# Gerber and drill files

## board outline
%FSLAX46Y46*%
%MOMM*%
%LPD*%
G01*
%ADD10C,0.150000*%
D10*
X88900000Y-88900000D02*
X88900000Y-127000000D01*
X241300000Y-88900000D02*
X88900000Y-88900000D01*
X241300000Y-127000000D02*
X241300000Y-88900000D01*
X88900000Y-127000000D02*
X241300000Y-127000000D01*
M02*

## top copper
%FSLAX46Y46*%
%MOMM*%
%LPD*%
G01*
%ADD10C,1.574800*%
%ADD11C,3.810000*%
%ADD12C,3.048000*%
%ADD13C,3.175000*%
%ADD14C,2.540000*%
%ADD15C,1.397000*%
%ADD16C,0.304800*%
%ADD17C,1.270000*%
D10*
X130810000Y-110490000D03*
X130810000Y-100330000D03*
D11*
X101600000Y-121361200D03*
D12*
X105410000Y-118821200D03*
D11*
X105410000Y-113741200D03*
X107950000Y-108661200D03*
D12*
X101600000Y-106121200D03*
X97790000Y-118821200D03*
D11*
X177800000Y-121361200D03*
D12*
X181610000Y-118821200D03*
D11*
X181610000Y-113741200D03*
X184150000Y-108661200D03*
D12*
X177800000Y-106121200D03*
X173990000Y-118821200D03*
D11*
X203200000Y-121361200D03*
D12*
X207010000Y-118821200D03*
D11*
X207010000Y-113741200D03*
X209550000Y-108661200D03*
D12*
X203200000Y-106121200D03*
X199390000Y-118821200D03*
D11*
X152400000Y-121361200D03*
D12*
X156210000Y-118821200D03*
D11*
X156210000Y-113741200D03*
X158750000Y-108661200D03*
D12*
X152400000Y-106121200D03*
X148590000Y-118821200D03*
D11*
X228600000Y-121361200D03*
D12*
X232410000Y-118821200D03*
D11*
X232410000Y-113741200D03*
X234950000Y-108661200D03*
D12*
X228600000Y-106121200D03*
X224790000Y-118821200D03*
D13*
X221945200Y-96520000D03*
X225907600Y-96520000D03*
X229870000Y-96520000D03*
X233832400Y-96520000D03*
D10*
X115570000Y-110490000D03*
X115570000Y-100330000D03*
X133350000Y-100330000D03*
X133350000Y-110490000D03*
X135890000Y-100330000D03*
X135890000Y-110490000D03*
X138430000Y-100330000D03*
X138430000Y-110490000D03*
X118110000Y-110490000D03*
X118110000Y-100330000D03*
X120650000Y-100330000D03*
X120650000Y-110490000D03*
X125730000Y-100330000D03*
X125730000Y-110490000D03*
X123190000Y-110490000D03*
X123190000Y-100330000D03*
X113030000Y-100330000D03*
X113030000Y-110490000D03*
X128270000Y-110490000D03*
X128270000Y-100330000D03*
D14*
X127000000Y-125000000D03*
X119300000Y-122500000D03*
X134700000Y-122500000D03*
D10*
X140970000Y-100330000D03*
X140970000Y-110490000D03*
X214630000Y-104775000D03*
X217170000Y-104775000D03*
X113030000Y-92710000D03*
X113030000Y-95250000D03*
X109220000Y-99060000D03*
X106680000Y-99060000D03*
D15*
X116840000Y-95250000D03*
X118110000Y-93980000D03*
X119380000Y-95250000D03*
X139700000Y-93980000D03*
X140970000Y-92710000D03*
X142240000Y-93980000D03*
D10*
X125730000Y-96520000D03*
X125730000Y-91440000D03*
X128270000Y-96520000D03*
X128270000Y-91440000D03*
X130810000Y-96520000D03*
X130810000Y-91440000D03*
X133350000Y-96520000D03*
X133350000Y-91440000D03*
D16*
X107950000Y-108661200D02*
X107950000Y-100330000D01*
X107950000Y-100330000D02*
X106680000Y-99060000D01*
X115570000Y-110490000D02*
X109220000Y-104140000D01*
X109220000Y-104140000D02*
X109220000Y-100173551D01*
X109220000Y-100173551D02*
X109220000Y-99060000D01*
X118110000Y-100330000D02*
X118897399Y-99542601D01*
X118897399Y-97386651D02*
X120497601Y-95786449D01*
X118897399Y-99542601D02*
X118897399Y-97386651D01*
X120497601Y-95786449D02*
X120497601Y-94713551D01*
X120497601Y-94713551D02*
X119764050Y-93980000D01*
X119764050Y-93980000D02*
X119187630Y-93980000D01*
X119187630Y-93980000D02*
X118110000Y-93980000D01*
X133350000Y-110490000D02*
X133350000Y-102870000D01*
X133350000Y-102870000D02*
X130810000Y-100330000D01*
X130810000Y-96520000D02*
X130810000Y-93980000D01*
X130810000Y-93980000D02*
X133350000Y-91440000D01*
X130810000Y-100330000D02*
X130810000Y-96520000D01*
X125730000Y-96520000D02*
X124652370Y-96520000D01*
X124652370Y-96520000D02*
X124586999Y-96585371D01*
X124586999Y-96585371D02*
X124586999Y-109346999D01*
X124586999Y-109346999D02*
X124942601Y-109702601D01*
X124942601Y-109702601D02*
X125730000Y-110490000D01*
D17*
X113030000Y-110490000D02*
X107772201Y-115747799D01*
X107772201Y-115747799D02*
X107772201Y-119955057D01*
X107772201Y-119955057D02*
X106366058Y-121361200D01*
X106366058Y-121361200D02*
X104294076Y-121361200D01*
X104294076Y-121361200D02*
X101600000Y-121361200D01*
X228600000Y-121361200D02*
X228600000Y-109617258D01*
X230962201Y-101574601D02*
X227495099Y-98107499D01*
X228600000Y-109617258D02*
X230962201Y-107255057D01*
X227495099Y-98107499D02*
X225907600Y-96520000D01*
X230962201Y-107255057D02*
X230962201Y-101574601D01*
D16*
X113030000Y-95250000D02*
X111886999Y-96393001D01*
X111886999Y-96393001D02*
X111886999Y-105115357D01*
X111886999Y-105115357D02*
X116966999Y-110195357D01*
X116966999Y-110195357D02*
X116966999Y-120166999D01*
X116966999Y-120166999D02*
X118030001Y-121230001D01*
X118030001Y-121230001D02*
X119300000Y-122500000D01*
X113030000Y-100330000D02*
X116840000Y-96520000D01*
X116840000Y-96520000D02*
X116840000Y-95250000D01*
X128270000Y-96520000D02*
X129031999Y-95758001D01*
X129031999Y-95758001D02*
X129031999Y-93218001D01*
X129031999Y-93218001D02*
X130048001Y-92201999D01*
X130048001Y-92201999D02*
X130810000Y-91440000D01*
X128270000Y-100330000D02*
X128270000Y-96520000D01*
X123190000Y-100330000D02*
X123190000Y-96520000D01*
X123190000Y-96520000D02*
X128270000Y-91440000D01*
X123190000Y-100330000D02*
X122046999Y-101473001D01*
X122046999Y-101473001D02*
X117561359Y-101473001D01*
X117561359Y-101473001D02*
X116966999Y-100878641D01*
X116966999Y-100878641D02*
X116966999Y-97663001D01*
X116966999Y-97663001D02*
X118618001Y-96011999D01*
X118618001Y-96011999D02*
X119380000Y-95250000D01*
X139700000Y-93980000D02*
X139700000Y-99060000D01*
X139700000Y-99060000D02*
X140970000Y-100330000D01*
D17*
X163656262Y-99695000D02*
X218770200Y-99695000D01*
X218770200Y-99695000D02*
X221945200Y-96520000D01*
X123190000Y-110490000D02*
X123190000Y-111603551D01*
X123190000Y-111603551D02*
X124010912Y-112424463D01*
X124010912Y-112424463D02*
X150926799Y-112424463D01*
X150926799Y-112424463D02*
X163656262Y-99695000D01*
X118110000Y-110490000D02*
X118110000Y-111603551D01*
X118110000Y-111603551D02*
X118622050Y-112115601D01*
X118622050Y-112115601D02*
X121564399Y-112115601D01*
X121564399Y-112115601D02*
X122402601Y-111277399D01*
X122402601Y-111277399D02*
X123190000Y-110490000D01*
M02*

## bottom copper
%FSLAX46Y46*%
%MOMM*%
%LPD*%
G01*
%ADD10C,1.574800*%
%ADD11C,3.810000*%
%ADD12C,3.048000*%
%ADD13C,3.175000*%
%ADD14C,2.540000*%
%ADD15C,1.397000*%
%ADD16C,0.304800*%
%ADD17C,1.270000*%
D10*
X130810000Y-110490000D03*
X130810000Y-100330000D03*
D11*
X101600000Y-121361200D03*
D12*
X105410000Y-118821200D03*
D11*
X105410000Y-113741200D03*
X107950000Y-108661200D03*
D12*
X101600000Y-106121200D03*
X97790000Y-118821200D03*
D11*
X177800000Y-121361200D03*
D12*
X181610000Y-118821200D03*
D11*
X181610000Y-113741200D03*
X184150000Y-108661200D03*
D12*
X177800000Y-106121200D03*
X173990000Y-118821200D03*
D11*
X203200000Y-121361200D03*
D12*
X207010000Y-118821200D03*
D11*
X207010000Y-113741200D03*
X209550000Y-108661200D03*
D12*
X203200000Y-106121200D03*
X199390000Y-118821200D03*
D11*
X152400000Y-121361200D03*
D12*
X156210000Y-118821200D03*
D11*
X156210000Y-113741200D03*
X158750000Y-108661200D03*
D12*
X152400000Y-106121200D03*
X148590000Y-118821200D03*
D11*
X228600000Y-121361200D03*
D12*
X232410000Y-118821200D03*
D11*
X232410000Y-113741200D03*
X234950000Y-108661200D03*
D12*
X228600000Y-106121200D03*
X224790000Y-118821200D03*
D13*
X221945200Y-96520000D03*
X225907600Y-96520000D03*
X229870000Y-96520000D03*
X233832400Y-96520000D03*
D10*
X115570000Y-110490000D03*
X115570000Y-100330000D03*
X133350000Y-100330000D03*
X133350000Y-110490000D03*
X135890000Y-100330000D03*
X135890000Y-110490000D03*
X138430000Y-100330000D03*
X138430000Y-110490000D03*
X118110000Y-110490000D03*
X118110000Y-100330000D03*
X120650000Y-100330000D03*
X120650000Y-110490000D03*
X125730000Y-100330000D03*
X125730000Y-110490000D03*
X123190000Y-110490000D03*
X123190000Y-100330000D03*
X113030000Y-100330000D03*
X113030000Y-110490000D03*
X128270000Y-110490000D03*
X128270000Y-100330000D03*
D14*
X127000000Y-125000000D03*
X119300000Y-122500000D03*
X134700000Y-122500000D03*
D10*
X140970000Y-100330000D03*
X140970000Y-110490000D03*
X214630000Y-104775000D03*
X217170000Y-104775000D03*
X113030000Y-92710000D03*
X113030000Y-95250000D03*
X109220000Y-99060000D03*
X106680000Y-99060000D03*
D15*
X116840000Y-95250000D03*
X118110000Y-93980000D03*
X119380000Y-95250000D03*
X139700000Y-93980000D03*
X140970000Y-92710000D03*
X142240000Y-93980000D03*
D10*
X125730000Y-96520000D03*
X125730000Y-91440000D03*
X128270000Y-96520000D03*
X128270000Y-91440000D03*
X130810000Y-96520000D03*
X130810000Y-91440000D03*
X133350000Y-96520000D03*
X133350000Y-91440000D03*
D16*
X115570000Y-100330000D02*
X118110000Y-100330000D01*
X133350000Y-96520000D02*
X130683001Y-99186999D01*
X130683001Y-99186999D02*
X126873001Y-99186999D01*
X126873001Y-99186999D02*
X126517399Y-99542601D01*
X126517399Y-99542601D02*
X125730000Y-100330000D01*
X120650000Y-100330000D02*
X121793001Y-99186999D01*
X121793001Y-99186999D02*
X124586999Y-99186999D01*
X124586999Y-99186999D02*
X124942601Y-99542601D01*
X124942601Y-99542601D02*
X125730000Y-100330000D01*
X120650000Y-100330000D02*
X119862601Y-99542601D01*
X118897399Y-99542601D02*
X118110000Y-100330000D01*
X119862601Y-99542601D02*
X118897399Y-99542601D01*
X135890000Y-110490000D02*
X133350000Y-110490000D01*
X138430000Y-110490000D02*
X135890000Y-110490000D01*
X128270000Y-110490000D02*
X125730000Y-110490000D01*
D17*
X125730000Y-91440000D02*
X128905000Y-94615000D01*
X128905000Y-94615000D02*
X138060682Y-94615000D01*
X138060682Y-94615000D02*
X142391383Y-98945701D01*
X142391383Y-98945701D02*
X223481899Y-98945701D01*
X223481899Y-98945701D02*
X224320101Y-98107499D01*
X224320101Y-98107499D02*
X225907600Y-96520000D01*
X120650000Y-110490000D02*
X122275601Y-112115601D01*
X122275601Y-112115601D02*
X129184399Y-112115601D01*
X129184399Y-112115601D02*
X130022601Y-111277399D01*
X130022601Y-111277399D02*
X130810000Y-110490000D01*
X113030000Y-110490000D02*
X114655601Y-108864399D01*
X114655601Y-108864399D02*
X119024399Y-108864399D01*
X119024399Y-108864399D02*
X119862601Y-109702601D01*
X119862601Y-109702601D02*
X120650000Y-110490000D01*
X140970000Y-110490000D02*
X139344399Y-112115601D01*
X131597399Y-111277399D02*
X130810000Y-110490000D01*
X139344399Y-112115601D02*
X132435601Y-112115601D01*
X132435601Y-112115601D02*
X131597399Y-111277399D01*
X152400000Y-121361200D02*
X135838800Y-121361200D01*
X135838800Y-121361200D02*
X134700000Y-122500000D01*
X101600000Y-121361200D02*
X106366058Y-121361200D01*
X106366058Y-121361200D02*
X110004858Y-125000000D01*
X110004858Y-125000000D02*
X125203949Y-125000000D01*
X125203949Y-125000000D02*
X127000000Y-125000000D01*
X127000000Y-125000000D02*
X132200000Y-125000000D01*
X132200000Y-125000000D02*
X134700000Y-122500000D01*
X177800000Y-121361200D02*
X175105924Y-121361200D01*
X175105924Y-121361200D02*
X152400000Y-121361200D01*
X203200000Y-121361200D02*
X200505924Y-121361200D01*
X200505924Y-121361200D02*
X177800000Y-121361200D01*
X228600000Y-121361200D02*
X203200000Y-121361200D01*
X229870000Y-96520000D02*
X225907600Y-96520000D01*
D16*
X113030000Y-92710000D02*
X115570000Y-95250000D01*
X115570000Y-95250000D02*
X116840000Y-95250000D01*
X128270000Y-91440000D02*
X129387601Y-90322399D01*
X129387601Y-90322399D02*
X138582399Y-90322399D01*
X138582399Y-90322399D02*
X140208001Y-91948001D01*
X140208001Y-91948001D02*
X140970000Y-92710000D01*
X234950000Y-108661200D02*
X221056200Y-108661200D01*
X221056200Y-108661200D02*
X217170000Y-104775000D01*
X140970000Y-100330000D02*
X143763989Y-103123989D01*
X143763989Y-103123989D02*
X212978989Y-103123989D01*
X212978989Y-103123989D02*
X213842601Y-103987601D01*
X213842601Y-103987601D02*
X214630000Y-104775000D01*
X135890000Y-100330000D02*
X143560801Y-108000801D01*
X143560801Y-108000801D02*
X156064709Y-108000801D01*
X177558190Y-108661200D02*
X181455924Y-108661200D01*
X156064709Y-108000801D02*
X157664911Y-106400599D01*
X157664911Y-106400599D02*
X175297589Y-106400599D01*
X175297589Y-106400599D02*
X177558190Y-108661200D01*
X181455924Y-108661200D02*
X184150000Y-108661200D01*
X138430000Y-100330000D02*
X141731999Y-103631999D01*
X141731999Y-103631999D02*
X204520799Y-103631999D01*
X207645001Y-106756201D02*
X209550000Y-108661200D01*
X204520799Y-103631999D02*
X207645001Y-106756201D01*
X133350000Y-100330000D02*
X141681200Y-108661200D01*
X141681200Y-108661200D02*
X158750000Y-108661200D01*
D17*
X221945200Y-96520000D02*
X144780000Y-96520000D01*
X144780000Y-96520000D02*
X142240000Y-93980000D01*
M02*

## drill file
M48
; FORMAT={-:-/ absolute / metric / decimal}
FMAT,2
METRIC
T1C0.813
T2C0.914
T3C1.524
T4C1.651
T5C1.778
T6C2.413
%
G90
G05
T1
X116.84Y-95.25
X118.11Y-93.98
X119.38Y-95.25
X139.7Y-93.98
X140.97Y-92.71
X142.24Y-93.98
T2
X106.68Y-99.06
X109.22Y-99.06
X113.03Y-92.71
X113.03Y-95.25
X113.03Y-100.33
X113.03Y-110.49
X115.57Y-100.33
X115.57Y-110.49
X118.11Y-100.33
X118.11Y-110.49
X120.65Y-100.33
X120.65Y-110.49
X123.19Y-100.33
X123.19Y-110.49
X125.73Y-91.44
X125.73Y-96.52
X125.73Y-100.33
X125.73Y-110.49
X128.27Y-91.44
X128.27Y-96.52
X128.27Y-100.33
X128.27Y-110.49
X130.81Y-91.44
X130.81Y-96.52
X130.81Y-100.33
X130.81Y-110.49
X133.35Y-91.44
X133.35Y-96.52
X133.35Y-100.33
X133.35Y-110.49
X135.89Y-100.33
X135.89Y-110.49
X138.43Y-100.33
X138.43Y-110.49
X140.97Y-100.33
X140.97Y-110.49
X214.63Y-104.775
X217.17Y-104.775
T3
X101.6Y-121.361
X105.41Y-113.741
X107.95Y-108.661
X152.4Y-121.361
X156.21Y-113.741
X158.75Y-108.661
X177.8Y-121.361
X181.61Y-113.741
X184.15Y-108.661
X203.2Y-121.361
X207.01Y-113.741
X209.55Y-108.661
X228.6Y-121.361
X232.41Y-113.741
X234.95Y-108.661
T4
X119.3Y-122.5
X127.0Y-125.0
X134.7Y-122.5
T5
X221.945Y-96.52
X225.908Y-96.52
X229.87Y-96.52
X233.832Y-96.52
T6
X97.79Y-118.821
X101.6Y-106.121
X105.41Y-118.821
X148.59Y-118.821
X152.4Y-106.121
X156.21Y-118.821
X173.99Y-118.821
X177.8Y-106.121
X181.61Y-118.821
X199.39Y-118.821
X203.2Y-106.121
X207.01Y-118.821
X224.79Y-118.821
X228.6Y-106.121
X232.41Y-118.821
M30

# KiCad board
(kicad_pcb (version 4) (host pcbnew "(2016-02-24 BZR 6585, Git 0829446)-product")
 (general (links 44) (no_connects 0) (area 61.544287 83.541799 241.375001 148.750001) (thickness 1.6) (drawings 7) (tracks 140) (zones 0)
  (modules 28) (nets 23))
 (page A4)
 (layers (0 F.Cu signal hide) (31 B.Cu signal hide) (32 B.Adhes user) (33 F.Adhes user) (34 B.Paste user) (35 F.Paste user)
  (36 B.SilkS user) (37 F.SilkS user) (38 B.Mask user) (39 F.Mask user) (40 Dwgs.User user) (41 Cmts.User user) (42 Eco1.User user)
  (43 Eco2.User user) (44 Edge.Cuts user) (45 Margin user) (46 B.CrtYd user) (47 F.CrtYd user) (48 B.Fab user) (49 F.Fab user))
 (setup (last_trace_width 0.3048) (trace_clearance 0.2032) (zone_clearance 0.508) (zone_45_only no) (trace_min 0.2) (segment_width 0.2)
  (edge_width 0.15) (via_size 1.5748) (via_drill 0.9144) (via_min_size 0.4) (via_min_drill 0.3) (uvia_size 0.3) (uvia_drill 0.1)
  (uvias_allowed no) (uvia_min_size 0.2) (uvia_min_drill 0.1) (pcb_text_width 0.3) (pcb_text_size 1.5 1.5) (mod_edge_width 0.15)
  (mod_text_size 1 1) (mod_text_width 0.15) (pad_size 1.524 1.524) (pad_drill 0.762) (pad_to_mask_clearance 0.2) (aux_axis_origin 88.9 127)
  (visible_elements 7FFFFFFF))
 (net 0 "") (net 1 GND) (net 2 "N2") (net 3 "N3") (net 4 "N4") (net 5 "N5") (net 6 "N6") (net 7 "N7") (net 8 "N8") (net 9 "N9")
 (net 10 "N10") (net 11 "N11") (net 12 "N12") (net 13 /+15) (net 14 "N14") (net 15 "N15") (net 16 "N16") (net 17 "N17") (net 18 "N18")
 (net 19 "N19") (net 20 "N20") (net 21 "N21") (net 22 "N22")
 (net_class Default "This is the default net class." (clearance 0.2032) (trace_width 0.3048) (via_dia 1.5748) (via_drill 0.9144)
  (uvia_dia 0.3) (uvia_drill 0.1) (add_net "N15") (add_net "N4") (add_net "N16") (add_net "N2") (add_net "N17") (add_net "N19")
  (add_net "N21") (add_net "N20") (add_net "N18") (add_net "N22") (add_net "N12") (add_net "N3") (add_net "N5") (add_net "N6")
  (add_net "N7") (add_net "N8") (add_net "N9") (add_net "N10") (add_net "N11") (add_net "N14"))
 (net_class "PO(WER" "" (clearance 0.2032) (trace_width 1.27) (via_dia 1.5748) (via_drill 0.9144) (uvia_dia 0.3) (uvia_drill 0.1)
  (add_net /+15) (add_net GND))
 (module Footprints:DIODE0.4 (layer F.Cu) (at 130.81 105.41 90)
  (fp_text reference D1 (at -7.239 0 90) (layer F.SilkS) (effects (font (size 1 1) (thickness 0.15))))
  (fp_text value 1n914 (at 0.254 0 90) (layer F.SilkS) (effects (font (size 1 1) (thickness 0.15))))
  (pad 1 thru_hole circle (at -5.08 0 90) (size 1.5748 1.5748) (drill 0.9144) (layers *.Cu *.Mask F.SilkS) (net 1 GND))
  (pad 2 thru_hole circle (at 5.08 0 90) (size 1.5748 1.5748) (drill 0.9144) (layers *.Cu *.Mask F.SilkS) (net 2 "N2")))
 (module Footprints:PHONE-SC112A (layer F.Cu) (at 101.6 127 270)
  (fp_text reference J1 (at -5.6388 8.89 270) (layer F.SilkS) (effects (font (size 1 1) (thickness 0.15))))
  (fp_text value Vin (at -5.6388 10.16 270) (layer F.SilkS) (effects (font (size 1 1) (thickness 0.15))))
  (pad 1 thru_hole circle (at -5.6388 0 270) (size 3.81 3.81) (drill 1.524) (layers *.Cu *.Mask F.SilkS) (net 1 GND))
  (pad "" thru_hole circle (at -8.1788 -3.81 270) (size 3.048 3.048) (drill 2.413) (layers *.Cu *.Mask F.SilkS))
  (pad 2 thru_hole circle (at -13.2588 -3.81 270) (size 3.81 3.81) (drill 1.524) (layers *.Cu *.Mask F.SilkS) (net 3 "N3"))
  (pad 3 thru_hole circle (at -18.3388 -6.35 270) (size 3.81 3.81) (drill 1.524) (layers *.Cu *.Mask F.SilkS) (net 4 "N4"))
  (pad "" thru_hole circle (at -20.8788 0 270) (size 3.048 3.048) (drill 2.413) (layers *.Cu *.Mask F.SilkS))
  (pad "" thru_hole circle (at -8.1788 3.81 270) (size 3.048 3.048) (drill 2.413) (layers *.Cu *.Mask F.SilkS)))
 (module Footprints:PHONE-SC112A (layer F.Cu) (at 177.8 127 270)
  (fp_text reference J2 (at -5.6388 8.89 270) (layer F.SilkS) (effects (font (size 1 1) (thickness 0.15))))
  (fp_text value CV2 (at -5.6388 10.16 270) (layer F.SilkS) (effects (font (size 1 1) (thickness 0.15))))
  (pad 1 thru_hole circle (at -5.6388 0 270) (size 3.81 3.81) (drill 1.524) (layers *.Cu *.Mask F.SilkS) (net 1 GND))
  (pad "" thru_hole circle (at -8.1788 -3.81 270) (size 3.048 3.048) (drill 2.413) (layers *.Cu *.Mask F.SilkS))
  (pad 2 thru_hole circle (at -13.2588 -3.81 270) (size 3.81 3.81) (drill 1.524) (layers *.Cu *.Mask F.SilkS) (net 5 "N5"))
  (pad 3 thru_hole circle (at -18.3388 -6.35 270) (size 3.81 3.81) (drill 1.524) (layers *.Cu *.Mask F.SilkS) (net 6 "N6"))
  (pad "" thru_hole circle (at -20.8788 0 270) (size 3.048 3.048) (drill 2.413) (layers *.Cu *.Mask F.SilkS))
  (pad "" thru_hole circle (at -8.1788 3.81 270) (size 3.048 3.048) (drill 2.413) (layers *.Cu *.Mask F.SilkS)))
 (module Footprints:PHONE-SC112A (layer F.Cu) (at 203.2 127 270)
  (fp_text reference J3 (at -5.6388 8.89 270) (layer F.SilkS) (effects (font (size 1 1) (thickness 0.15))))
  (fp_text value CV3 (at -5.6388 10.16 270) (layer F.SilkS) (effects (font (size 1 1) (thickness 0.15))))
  (pad 1 thru_hole circle (at -5.6388 0 270) (size 3.81 3.81) (drill 1.524) (layers *.Cu *.Mask F.SilkS) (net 1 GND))
  (pad "" thru_hole circle (at -8.1788 -3.81 270) (size 3.048 3.048) (drill 2.413) (layers *.Cu *.Mask F.SilkS))
  (pad 2 thru_hole circle (at -13.2588 -3.81 270) (size 3.81 3.81) (drill 1.524) (layers *.Cu *.Mask F.SilkS) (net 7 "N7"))
  (pad 3 thru_hole circle (at -18.3388 -6.35 270) (size 3.81 3.81) (drill 1.524) (layers *.Cu *.Mask F.SilkS) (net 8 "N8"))
  (pad "" thru_hole circle (at -20.8788 0 270) (size 3.048 3.048) (drill 2.413) (layers *.Cu *.Mask F.SilkS))
  (pad "" thru_hole circle (at -8.1788 3.81 270) (size 3.048 3.048) (drill 2.413) (layers *.Cu *.Mask F.SilkS)))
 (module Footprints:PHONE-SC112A (layer F.Cu) (at 152.4 127 270)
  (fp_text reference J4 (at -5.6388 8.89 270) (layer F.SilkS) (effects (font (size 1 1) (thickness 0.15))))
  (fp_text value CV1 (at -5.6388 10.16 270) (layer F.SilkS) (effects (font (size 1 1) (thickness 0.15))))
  (pad 1 thru_hole circle (at -5.6388 0 270) (size 3.81 3.81) (drill 1.524) (layers *.Cu *.Mask F.SilkS) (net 1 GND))
  (pad "" thru_hole circle (at -8.1788 -3.81 270) (size 3.048 3.048) (drill 2.413) (layers *.Cu *.Mask F.SilkS))
  (pad 2 thru_hole circle (at -13.2588 -3.81 270) (size 3.81 3.81) (drill 1.524) (layers *.Cu *.Mask F.SilkS) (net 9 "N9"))
  (pad 3 thru_hole circle (at -18.3388 -6.35 270) (size 3.81 3.81) (drill 1.524) (layers *.Cu *.Mask F.SilkS) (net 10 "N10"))
  (pad "" thru_hole circle (at -20.8788 0 270) (size 3.048 3.048) (drill 2.413) (layers *.Cu *.Mask F.SilkS))
  (pad "" thru_hole circle (at -8.1788 3.81 270) (size 3.048 3.048) (drill 2.413) (layers *.Cu *.Mask F.SilkS)))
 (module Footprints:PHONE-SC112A (layer F.Cu) (at 228.6 127 270)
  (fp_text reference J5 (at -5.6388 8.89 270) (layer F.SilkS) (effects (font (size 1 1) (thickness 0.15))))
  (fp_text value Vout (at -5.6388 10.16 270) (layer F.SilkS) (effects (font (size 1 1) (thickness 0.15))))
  (pad 1 thru_hole circle (at -5.6388 0 270) (size 3.81 3.81) (drill 1.524) (layers *.Cu *.Mask F.SilkS) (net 1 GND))
  (pad "" thru_hole circle (at -8.1788 -3.81 270) (size 3.048 3.048) (drill 2.413) (layers *.Cu *.Mask F.SilkS))
  (pad 2 thru_hole circle (at -13.2588 -3.81 270) (size 3.81 3.81) (drill 1.524) (layers *.Cu *.Mask F.SilkS) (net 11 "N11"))
  (pad 3 thru_hole circle (at -18.3388 -6.35 270) (size 3.81 3.81) (drill 1.524) (layers *.Cu *.Mask F.SilkS) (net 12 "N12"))
  (pad "" thru_hole circle (at -20.8788 0 270) (size 3.048 3.048) (drill 2.413) (layers *.Cu *.Mask F.SilkS))
  (pad "" thru_hole circle (at -8.1788 3.81 270) (size 3.048 3.048) (drill 2.413) (layers *.Cu *.Mask F.SilkS)))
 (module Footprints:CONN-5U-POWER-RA (layer F.Cu) (at 227.8888 96.52)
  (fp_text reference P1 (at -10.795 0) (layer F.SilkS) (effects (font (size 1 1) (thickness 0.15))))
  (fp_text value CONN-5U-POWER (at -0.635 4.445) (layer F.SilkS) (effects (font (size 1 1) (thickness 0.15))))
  (pad 1 thru_hole circle (at -5.9436 0) (size 3.175 3.175) (drill 1.778) (layers *.Cu *.Mask F.SilkS) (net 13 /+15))
  (pad 2 thru_hole circle (at -1.9812 0) (size 3.175 3.175) (drill 1.778) (layers *.Cu *.Mask F.SilkS) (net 1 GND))
  (pad 3 thru_hole circle (at 1.9812 0) (size 3.175 3.175) (drill 1.778) (layers *.Cu *.Mask F.SilkS) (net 1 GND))
  (pad 4 thru_hole circle (at 5.9436 0) (size 3.175 3.175) (drill 1.778) (layers *.Cu *.Mask F.SilkS) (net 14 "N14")))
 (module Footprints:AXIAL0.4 (layer F.Cu) (at 115.57 105.41 90)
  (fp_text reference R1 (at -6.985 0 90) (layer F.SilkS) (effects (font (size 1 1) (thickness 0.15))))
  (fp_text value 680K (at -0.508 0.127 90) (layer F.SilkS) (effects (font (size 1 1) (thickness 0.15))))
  (pad 1 thru_hole circle (at -5.08 0 90) (size 1.5748 1.5748) (drill 0.9144) (layers *.Cu *.Mask F.SilkS) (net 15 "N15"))
  (pad 2 thru_hole circle (at 5.08 0 90) (size 1.5748 1.5748) (drill 0.9144) (layers *.Cu *.Mask F.SilkS) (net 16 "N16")))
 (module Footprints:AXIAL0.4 (layer F.Cu) (at 133.35 105.41 270)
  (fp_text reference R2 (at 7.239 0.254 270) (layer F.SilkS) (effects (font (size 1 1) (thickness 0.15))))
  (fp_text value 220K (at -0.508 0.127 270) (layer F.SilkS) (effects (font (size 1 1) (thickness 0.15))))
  (pad 1 thru_hole circle (at -5.08 0 270) (size 1.5748 1.5748) (drill 0.9144) (layers *.Cu *.Mask F.SilkS) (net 10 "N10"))
  (pad 2 thru_hole circle (at 5.08 0 270) (size 1.5748 1.5748) (drill 0.9144) (layers *.Cu *.Mask F.SilkS) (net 2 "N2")))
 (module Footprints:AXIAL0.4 (layer F.Cu) (at 135.89 105.41 270)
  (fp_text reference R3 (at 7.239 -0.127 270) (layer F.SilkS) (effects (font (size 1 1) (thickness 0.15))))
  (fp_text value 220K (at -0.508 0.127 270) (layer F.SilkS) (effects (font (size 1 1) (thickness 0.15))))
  (pad 1 thru_hole circle (at -5.08 0 270) (size 1.5748 1.5748) (drill 0.9144) (layers *.Cu *.Mask F.SilkS) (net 6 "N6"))
  (pad 2 thru_hole circle (at 5.08 0 270) (size 1.5748 1.5748) (drill 0.9144) (layers *.Cu *.Mask F.SilkS) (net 2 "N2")))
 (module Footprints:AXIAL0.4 (layer F.Cu) (at 138.43 105.41 270)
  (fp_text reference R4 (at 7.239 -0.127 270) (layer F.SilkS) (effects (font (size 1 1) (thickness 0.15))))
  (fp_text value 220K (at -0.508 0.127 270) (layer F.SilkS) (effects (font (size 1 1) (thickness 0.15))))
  (pad 1 thru_hole circle (at -5.08 0 270) (size 1.5748 1.5748) (drill 0.9144) (layers *.Cu *.Mask F.SilkS) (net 8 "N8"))
  (pad 2 thru_hole circle (at 5.08 0 270) (size 1.5748 1.5748) (drill 0.9144) (layers *.Cu *.Mask F.SilkS) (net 2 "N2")))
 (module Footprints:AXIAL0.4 (layer F.Cu) (at 118.11 105.41 90)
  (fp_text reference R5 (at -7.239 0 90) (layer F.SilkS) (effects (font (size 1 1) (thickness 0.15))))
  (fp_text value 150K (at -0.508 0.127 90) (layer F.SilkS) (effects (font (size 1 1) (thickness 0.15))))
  (pad 1 thru_hole circle (at -5.08 0 90) (size 1.5748 1.5748) (drill 0.9144) (layers *.Cu *.Mask F.SilkS) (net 13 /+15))
  (pad 2 thru_hole circle (at 5.08 0 90) (size 1.5748 1.5748) (drill 0.9144) (layers *.Cu *.Mask F.SilkS) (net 16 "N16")))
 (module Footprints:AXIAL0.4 (layer F.Cu) (at 120.65 105.41 270)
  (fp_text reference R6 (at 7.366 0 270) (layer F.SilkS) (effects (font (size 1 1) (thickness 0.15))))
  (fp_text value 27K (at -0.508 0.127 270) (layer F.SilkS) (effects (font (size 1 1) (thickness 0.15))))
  (pad 1 thru_hole circle (at -5.08 0 270) (size 1.5748 1.5748) (drill 0.9144) (layers *.Cu *.Mask F.SilkS) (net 16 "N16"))
  (pad 2 thru_hole circle (at 5.08 0 270) (size 1.5748 1.5748) (drill 0.9144) (layers *.Cu *.Mask F.SilkS) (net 1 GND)))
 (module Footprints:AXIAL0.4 (layer F.Cu) (at 125.73 105.41 270)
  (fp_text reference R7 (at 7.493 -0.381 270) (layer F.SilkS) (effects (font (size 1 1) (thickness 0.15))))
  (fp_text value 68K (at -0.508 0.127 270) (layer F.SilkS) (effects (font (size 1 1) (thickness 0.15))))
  (pad 1 thru_hole circle (at -5.08 0 270) (size 1.5748 1.5748) (drill 0.9144) (layers *.Cu *.Mask F.SilkS) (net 16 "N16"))
  (pad 2 thru_hole circle (at 5.08 0 270) (size 1.5748 1.5748) (drill 0.9144) (layers *.Cu *.Mask F.SilkS) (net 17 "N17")))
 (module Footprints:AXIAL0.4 (layer F.Cu) (at 123.19 105.41 90)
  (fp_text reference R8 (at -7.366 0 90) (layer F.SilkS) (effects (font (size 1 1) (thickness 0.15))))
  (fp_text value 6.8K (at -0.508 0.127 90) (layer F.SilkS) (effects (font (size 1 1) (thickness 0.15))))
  (pad 1 thru_hole circle (at -5.08 0 90) (size 1.5748 1.5748) (drill 0.9144) (layers *.Cu *.Mask F.SilkS) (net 13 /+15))
  (pad 2 thru_hole circle (at 5.08 0 90) (size 1.5748 1.5748) (drill 0.9144) (layers *.Cu *.Mask F.SilkS) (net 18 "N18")))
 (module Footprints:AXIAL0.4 (layer F.Cu) (at 113.03 105.41 270)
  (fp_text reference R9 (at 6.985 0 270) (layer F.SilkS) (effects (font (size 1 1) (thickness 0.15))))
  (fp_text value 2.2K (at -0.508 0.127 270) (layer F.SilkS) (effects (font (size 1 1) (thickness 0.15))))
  (pad 1 thru_hole circle (at -5.08 0 270) (size 1.5748 1.5748) (drill 0.9144) (layers *.Cu *.Mask F.SilkS) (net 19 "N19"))
  (pad 2 thru_hole circle (at 5.08 0 270) (size 1.5748 1.5748) (drill 0.9144) (layers *.Cu *.Mask F.SilkS) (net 1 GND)))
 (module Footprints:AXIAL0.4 (layer F.Cu) (at 128.27 105.41 90)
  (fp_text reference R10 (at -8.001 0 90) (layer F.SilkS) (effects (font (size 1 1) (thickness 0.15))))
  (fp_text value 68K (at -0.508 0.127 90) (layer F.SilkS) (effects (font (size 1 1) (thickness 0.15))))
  (pad 1 thru_hole circle (at -5.08 0 90) (size 1.5748 1.5748) (drill 0.9144) (layers *.Cu *.Mask F.SilkS) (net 17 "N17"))
  (pad 2 thru_hole circle (at 5.08 0 90) (size 1.5748 1.5748) (drill 0.9144) (layers *.Cu *.Mask F.SilkS) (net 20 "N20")))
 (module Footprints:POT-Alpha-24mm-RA (layer F.Cu) (at 127 127)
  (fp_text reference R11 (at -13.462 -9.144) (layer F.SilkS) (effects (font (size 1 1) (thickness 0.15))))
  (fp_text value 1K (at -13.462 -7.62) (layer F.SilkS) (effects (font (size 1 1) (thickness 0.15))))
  (pad 2 thru_hole circle (at 0 -2) (size 2.54 2.54) (drill 1.651) (layers *.Cu *.Mask F.SilkS) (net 1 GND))
  (pad 1 thru_hole circle (at -7.7 -4.5) (size 2.54 2.54) (drill 1.651) (layers *.Cu *.Mask F.SilkS) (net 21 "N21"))
  (pad 3 thru_hole circle (at 7.7 -4.5) (size 2.54 2.54) (drill 1.651) (layers *.Cu *.Mask F.SilkS) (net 1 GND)))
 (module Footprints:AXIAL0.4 (layer F.Cu) (at 140.97 105.41 270)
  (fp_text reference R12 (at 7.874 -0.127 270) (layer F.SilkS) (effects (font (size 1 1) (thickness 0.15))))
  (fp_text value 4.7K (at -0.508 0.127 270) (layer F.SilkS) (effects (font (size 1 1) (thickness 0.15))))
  (pad 1 thru_hole circle (at -5.08 0 270) (size 1.5748 1.5748) (drill 0.9144) (layers *.Cu *.Mask F.SilkS) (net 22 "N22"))
  (pad 2 thru_hole circle (at 5.08 0 270) (size 1.5748 1.5748) (drill 0.9144) (layers *.Cu *.Mask F.SilkS) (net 1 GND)))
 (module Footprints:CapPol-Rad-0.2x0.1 (layer F.Cu) (at 217.17 107.315)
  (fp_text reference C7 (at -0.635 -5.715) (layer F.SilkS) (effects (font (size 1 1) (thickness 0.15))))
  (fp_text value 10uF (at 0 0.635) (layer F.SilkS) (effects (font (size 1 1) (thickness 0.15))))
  (pad 1 thru_hole circle (at -2.54 -2.54) (size 1.5748 1.5748) (drill 0.9144) (layers *.Cu *.Mask F.SilkS) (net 22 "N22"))
  (pad 2 thru_hole circle (at 0 -2.54) (size 1.5748 1.5748) (drill 0.9144) (layers *.Cu *.Mask F.SilkS) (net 12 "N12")))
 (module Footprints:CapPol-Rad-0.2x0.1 (layer F.Cu) (at 110.49 95.25 270)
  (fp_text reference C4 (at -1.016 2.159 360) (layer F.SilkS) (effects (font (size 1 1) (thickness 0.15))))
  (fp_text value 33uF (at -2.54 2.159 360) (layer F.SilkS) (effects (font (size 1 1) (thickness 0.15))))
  (pad 1 thru_hole circle (at -2.54 -2.54 270) (size 1.5748 1.5748) (drill 0.9144) (layers *.Cu *.Mask F.SilkS) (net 19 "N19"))
  (pad 2 thru_hole circle (at 0 -2.54 270) (size 1.5748 1.5748) (drill 0.9144) (layers *.Cu *.Mask F.SilkS) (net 21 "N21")))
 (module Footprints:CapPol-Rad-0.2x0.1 (layer F.Cu) (at 106.68 96.52 180)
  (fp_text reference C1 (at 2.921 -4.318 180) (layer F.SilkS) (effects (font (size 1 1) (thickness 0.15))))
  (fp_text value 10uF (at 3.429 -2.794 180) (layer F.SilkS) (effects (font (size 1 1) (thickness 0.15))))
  (pad 1 thru_hole circle (at -2.54 -2.54 180) (size 1.5748 1.5748) (drill 0.9144) (layers *.Cu *.Mask F.SilkS) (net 15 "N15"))
  (pad 2 thru_hole circle (at 0 -2.54 180) (size 1.5748 1.5748) (drill 0.9144) (layers *.Cu *.Mask F.SilkS) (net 4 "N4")))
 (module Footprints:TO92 (layer F.Cu) (at 118.11 97.79)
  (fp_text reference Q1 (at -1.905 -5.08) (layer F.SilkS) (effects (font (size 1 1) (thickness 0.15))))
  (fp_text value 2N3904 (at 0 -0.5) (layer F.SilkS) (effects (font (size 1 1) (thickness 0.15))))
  (pad 1 thru_hole circle (at -1.27 -2.54) (size 1.397 1.397) (drill 0.8128) (layers *.Cu *.Mask F.SilkS) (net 19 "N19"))
  (pad 2 thru_hole circle (at 0 -3.81) (size 1.397 1.397) (drill 0.8128) (layers *.Cu *.Mask F.SilkS) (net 16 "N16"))
  (pad 3 thru_hole circle (at 1.27 -2.54) (size 1.397 1.397) (drill 0.8128) (layers *.Cu *.Mask F.SilkS) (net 18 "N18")))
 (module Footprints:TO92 (layer F.Cu) (at 140.97 96.52)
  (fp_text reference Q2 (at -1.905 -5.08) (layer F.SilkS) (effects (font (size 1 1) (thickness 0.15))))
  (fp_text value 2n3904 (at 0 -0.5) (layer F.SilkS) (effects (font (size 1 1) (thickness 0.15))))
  (pad 1 thru_hole circle (at -1.27 -2.54) (size 1.397 1.397) (drill 0.8128) (layers *.Cu *.Mask F.SilkS) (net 22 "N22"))
  (pad 2 thru_hole circle (at 0 -3.81) (size 1.397 1.397) (drill 0.8128) (layers *.Cu *.Mask F.SilkS) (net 18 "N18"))
  (pad 3 thru_hole circle (at 1.27 -2.54) (size 1.397 1.397) (drill 0.8128) (layers *.Cu *.Mask F.SilkS) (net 13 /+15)))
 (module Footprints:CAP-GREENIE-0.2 (layer F.Cu) (at 125.73 93.98 90)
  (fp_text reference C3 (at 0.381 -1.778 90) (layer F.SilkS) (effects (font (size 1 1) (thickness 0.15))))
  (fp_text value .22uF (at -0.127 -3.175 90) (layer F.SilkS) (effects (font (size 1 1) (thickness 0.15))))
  (pad 1 thru_hole circle (at -2.54 0 90) (size 1.5748 1.5748) (drill 0.9144) (layers *.Cu *.Mask F.SilkS) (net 17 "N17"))
  (pad 2 thru_hole circle (at 2.54 0 90) (size 1.5748 1.5748) (drill 0.9144) (layers *.Cu *.Mask F.SilkS) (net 1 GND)))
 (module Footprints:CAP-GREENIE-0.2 (layer F.Cu) (at 128.27 93.98 90)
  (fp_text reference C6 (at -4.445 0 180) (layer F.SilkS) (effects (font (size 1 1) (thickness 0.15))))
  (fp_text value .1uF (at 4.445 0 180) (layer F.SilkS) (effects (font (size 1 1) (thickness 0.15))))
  (pad 1 thru_hole circle (at -2.54 0 90) (size 1.5748 1.5748) (drill 0.9144) (layers *.Cu *.Mask F.SilkS) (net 20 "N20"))
  (pad 2 thru_hole circle (at 2.54 0 90) (size 1.5748 1.5748) (drill 0.9144) (layers *.Cu *.Mask F.SilkS) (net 18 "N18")))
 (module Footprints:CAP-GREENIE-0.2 (layer F.Cu) (at 130.81 93.98 90)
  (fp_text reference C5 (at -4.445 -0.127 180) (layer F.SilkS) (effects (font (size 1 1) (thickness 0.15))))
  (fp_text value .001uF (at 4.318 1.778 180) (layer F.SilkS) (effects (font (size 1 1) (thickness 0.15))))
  (pad 1 thru_hole circle (at -2.54 0 90) (size 1.5748 1.5748) (drill 0.9144) (layers *.Cu *.Mask F.SilkS) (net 2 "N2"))
  (pad 2 thru_hole circle (at 2.54 0 90) (size 1.5748 1.5748) (drill 0.9144) (layers *.Cu *.Mask F.SilkS) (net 20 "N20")))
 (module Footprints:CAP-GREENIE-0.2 (layer F.Cu) (at 133.35 93.98 90)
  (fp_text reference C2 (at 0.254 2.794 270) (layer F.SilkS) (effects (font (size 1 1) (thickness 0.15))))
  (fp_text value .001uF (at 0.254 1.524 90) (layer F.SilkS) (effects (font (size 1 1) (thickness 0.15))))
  (pad 1 thru_hole circle (at -2.54 0 90) (size 1.5748 1.5748) (drill 0.9144) (layers *.Cu *.Mask F.SilkS) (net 16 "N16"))
  (pad 2 thru_hole circle (at 2.54 0 90) (size 1.5748 1.5748) (drill 0.9144) (layers *.Cu *.Mask F.SilkS) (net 2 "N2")))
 (gr_line (start 88.9 88.9) (end 88.9 127) (layer Edge.Cuts) (width 0.15))
 (gr_line (start 241.3 88.9) (end 88.9 88.9) (layer Edge.Cuts) (width 0.15))
 (gr_line (start 241.3 127) (end 241.3 88.9) (layer Edge.Cuts) (width 0.15))
 (gr_line (start 88.9 127) (end 241.3 127) (layer Edge.Cuts) (width 0.15))
 (segment (start 107.95 108.6612) (end 107.95 100.33) (width 0.3048) (layer F.Cu) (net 4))
 (segment (start 107.95 100.33) (end 106.68 99.06) (width 0.3048) (layer F.Cu) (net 4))
 (segment (start 115.57 110.49) (end 109.22 104.14) (width 0.3048) (layer F.Cu) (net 15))
 (segment (start 109.22 104.14) (end 109.22 100.173551) (width 0.3048) (layer F.Cu) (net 15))
 (segment (start 109.22 100.173551) (end 109.22 99.06) (width 0.3048) (layer F.Cu) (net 15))
 (segment (start 115.57 100.33) (end 118.11 100.33) (width 0.3048) (layer B.Cu) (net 16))
 (segment (start 133.35 96.52) (end 130.683001 99.186999) (width 0.3048) (layer B.Cu) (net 16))
 (segment (start 130.683001 99.186999) (end 126.873001 99.186999) (width 0.3048) (layer B.Cu) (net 16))
 (segment (start 126.873001 99.186999) (end 126.517399 99.542601) (width 0.3048) (layer B.Cu) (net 16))
 (segment (start 126.517399 99.542601) (end 125.73 100.33) (width 0.3048) (layer B.Cu) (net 16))
 (segment (start 120.65 100.33) (end 121.793001 99.186999) (width 0.3048) (layer B.Cu) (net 16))
 (segment (start 121.793001 99.186999) (end 124.586999 99.186999) (width 0.3048) (layer B.Cu) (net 16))
 (segment (start 124.586999 99.186999) (end 124.942601 99.542601) (width 0.3048) (layer B.Cu) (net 16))
 (segment (start 124.942601 99.542601) (end 125.73 100.33) (width 0.3048) (layer B.Cu) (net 16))
 (segment (start 120.65 100.33) (end 119.862601 99.542601) (width 0.3048) (layer B.Cu) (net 16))
 (segment (start 118.897399 99.542601) (end 118.11 100.33) (width 0.3048) (layer B.Cu) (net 16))
 (segment (start 119.862601 99.542601) (end 118.897399 99.542601) (width 0.3048) (layer B.Cu) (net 16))
 (segment (start 118.11 100.33) (end 118.897399 99.542601) (width 0.3048) (layer F.Cu) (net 16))
 (segment (start 118.897399 97.386651) (end 120.497601 95.786449) (width 0.3048) (layer F.Cu) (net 16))
 (segment (start 118.897399 99.542601) (end 118.897399 97.386651) (width 0.3048) (layer F.Cu) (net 16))
 (segment (start 120.497601 95.786449) (end 120.497601 94.713551) (width 0.3048) (layer F.Cu) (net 16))
 (segment (start 120.497601 94.713551) (end 119.76405 93.98) (width 0.3048) (layer F.Cu) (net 16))
 (segment (start 119.76405 93.98) (end 119.18763 93.98) (width 0.3048) (layer F.Cu) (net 16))
 (segment (start 119.18763 93.98) (end 118.11 93.98) (width 0.3048) (layer F.Cu) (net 16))
 (segment (start 133.35 110.49) (end 133.35 102.87) (width 0.3048) (layer F.Cu) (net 2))
 (segment (start 133.35 102.87) (end 130.81 100.33) (width 0.3048) (layer F.Cu) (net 2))
 (segment (start 135.89 110.49) (end 133.35 110.49) (width 0.3048) (layer B.Cu) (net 2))
 (segment (start 138.43 110.49) (end 135.89 110.49) (width 0.3048) (layer B.Cu) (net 2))
 (segment (start 130.81 96.52) (end 130.81 93.98) (width 0.3048) (layer F.Cu) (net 2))
 (segment (start 130.81 93.98) (end 133.35 91.44) (width 0.3048) (layer F.Cu) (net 2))
 (segment (start 130.81 100.33) (end 130.81 96.52) (width 0.3048) (layer F.Cu) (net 2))
 (segment (start 128.27 110.49) (end 125.73 110.49) (width 0.3048) (layer B.Cu) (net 17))
 (segment (start 125.73 96.52) (end 124.65237 96.52) (width 0.3048) (layer F.Cu) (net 17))
 (segment (start 124.65237 96.52) (end 124.586999 96.585371) (width 0.3048) (layer F.Cu) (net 17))
 (segment (start 124.586999 96.585371) (end 124.586999 109.346999) (width 0.3048) (layer F.Cu) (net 17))
 (segment (start 124.586999 109.346999) (end 124.942601 109.702601) (width 0.3048) (layer F.Cu) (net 17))
 (segment (start 124.942601 109.702601) (end 125.73 110.49) (width 0.3048) (layer F.Cu) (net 17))
 (segment (start 125.73 91.44) (end 128.905 94.615) (width 1.27) (layer B.Cu) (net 1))
 (segment (start 128.905 94.615) (end 138.060682 94.615) (width 1.27) (layer B.Cu) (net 1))
 (segment (start 138.060682 94.615) (end 142.391383 98.945701) (width 1.27) (layer B.Cu) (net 1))
 (segment (start 142.391383 98.945701) (end 223.481899 98.945701) (width 1.27) (layer B.Cu) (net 1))
 (segment (start 223.481899 98.945701) (end 224.320101 98.107499) (width 1.27) (layer B.Cu) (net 1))
 (segment (start 224.320101 98.107499) (end 225.9076 96.52) (width 1.27) (layer B.Cu) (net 1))
 (segment (start 113.03 110.49) (end 107.772201 115.747799) (width 1.27) (layer F.Cu) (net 1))
 (segment (start 107.772201 115.747799) (end 107.772201 119.955057) (width 1.27) (layer F.Cu) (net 1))
 (segment (start 107.772201 119.955057) (end 106.366058 121.3612) (width 1.27) (layer F.Cu) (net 1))
 (segment (start 106.366058 121.3612) (end 104.294076 121.3612) (width 1.27) (layer F.Cu) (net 1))
 (segment (start 104.294076 121.3612) (end 101.6 121.3612) (width 1.27) (layer F.Cu) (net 1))
 (segment (start 120.65 110.49) (end 122.275601 112.115601) (width 1.27) (layer B.Cu) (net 1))
 (segment (start 122.275601 112.115601) (end 129.184399 112.115601) (width 1.27) (layer B.Cu) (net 1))
 (segment (start 129.184399 112.115601) (end 130.022601 111.277399) (width 1.27) (layer B.Cu) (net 1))
 (segment (start 130.022601 111.277399) (end 130.81 110.49) (width 1.27) (layer B.Cu) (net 1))
 (segment (start 113.03 110.49) (end 114.655601 108.864399) (width 1.27) (layer B.Cu) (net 1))
 (segment (start 114.655601 108.864399) (end 119.024399 108.864399) (width 1.27) (layer B.Cu) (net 1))
 (segment (start 119.024399 108.864399) (end 119.862601 109.702601) (width 1.27) (layer B.Cu) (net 1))
 (segment (start 119.862601 109.702601) (end 120.65 110.49) (width 1.27) (layer B.Cu) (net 1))
 (segment (start 140.97 110.49) (end 139.344399 112.115601) (width 1.27) (layer B.Cu) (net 1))
 (segment (start 131.597399 111.277399) (end 130.81 110.49) (width 1.27) (layer B.Cu) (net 1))
 (segment (start 139.344399 112.115601) (end 132.435601 112.115601) (width 1.27) (layer B.Cu) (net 1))
 (segment (start 132.435601 112.115601) (end 131.597399 111.277399) (width 1.27) (layer B.Cu) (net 1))
 (segment (start 152.4 121.3612) (end 135.8388 121.3612) (width 1.27) (layer B.Cu) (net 1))
 (segment (start 135.8388 121.3612) (end 134.7 122.5) (width 1.27) (layer B.Cu) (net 1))
 (segment (start 101.6 121.3612) (end 106.366058 121.3612) (width 1.27) (layer B.Cu) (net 1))
 (segment (start 106.366058 121.3612) (end 110.004858 125) (width 1.27) (layer B.Cu) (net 1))
 (segment (start 110.004858 125) (end 125.203949 125) (width 1.27) (layer B.Cu) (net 1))
 (segment (start 125.203949 125) (end 127 125) (width 1.27) (layer B.Cu) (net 1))
 (segment (start 127 125) (end 132.2 125) (width 1.27) (layer B.Cu) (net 1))
 (segment (start 132.2 125) (end 134.7 122.5) (width 1.27) (layer B.Cu) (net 1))
 (segment (start 177.8 121.3612) (end 175.105924 121.3612) (width 1.27) (layer B.Cu) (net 1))
 (segment (start 175.105924 121.3612) (end 152.4 121.3612) (width 1.27) (layer B.Cu) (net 1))
 (segment (start 203.2 121.3612) (end 200.505924 121.3612) (width 1.27) (layer B.Cu) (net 1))
 (segment (start 200.505924 121.3612) (end 177.8 121.3612) (width 1.27) (layer B.Cu) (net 1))
 (segment (start 228.6 121.3612) (end 203.2 121.3612) (width 1.27) (layer B.Cu) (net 1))
 (segment (start 228.6 121.3612) (end 228.6 109.617258) (width 1.27) (layer F.Cu) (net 1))
 (segment (start 230.962201 101.574601) (end 227.495099 98.107499) (width 1.27) (layer F.Cu) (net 1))
 (segment (start 228.6 109.617258) (end 230.962201 107.255057) (width 1.27) (layer F.Cu) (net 1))
 (segment (start 227.495099 98.107499) (end 225.9076 96.52) (width 1.27) (layer F.Cu) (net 1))
 (segment (start 230.962201 107.255057) (end 230.962201 101.574601) (width 1.27) (layer F.Cu) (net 1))
 (segment (start 229.87 96.52) (end 225.9076 96.52) (width 1.27) (layer B.Cu) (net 1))
 (segment (start 113.03 95.25) (end 111.886999 96.393001) (width 0.3048) (layer F.Cu) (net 21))
 (segment (start 111.886999 96.393001) (end 111.886999 105.115357) (width 0.3048) (layer F.Cu) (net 21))
 (segment (start 111.886999 105.115357) (end 116.966999 110.195357) (width 0.3048) (layer F.Cu) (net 21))
 (segment (start 116.966999 110.195357) (end 116.966999 120.166999) (width 0.3048) (layer F.Cu) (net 21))
 (segment (start 116.966999 120.166999) (end 118.030001 121.230001) (width 0.3048) (layer F.Cu) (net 21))
 (segment (start 118.030001 121.230001) (end 119.3 122.5) (width 0.3048) (layer F.Cu) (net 21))
 (segment (start 113.03 92.71) (end 115.57 95.25) (width 0.3048) (layer B.Cu) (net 19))
 (segment (start 115.57 95.25) (end 116.84 95.25) (width 0.3048) (layer B.Cu) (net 19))
 (segment (start 113.03 100.33) (end 116.84 96.52) (width 0.3048) (layer F.Cu) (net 19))
 (segment (start 116.84 96.52) (end 116.84 95.25) (width 0.3048) (layer F.Cu) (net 19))
 (segment (start 128.27 96.52) (end 129.031999 95.758001) (width 0.3048) (layer F.Cu) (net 20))
 (segment (start 129.031999 95.758001) (end 129.031999 93.218001) (width 0.3048) (layer F.Cu) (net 20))
 (segment (start 129.031999 93.218001) (end 130.048001 92.201999) (width 0.3048) (layer F.Cu) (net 20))
 (segment (start 130.048001 92.201999) (end 130.81 91.44) (width 0.3048) (layer F.Cu) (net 20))
 (segment (start 128.27 100.33) (end 128.27 96.52) (width 0.3048) (layer F.Cu) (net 20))
 (segment (start 123.19 100.33) (end 123.19 96.52) (width 0.3048) (layer F.Cu) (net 18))
 (segment (start 123.19 96.52) (end 128.27 91.44) (width 0.3048) (layer F.Cu) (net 18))
 (segment (start 128.27 91.44) (end 129.387601 90.322399) (width 0.3048) (layer B.Cu) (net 18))
 (segment (start 129.387601 90.322399) (end 138.582399 90.322399) (width 0.3048) (layer B.Cu) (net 18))
 (segment (start 138.582399 90.322399) (end 140.208001 91.948001) (width 0.3048) (layer B.Cu) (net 18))
 (segment (start 140.208001 91.948001) (end 140.97 92.71) (width 0.3048) (layer B.Cu) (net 18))
 (segment (start 123.19 100.33) (end 122.046999 101.473001) (width 0.3048) (layer F.Cu) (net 18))
 (segment (start 122.046999 101.473001) (end 117.561359 101.473001) (width 0.3048) (layer F.Cu) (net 18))
 (segment (start 117.561359 101.473001) (end 116.966999 100.878641) (width 0.3048) (layer F.Cu) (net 18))
 (segment (start 116.966999 100.878641) (end 116.966999 97.663001) (width 0.3048) (layer F.Cu) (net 18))
 (segment (start 116.966999 97.663001) (end 118.618001 96.011999) (width 0.3048) (layer F.Cu) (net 18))
 (segment (start 118.618001 96.011999) (end 119.38 95.25) (width 0.3048) (layer F.Cu) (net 18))
 (segment (start 234.95 108.6612) (end 221.0562 108.6612) (width 0.3048) (layer B.Cu) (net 12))
 (segment (start 221.0562 108.6612) (end 217.17 104.775) (width 0.3048) (layer B.Cu) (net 12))
 (segment (start 140.97 100.33) (end 143.763989 103.123989) (width 0.3048) (layer B.Cu) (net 22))
 (segment (start 143.763989 103.123989) (end 212.978989 103.123989) (width 0.3048) (layer B.Cu) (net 22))
 (segment (start 212.978989 103.123989) (end 213.842601 103.987601) (width 0.3048) (layer B.Cu) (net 22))
 (segment (start 213.842601 103.987601) (end 214.63 104.775) (width 0.3048) (layer B.Cu) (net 22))
 (segment (start 139.7 93.98) (end 139.7 99.06) (width 0.3048) (layer F.Cu) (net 22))
 (segment (start 139.7 99.06) (end 140.97 100.33) (width 0.3048) (layer F.Cu) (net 22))
 (segment (start 135.89 100.33) (end 143.560801 108.000801) (width 0.3048) (layer B.Cu) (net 6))
 (segment (start 143.560801 108.000801) (end 156.064709 108.000801) (width 0.3048) (layer B.Cu) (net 6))
 (segment (start 177.55819 108.6612) (end 181.455924 108.6612) (width 0.3048) (layer B.Cu) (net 6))
 (segment (start 156.064709 108.000801) (end 157.664911 106.400599) (width 0.3048) (layer B.Cu) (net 6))
 (segment (start 157.664911 106.400599) (end 175.297589 106.400599) (width 0.3048) (layer B.Cu) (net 6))
 (segment (start 175.297589 106.400599) (end 177.55819 108.6612) (width 0.3048) (layer B.Cu) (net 6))
 (segment (start 181.455924 108.6612) (end 184.15 108.6612) (width 0.3048) (layer B.Cu) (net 6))
 (segment (start 138.43 100.33) (end 141.731999 103.631999) (width 0.3048) (layer B.Cu) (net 8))
 (segment (start 141.731999 103.631999) (end 204.520799 103.631999) (width 0.3048) (layer B.Cu) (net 8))
 (segment (start 207.645001 106.756201) (end 209.55 108.6612) (width 0.3048) (layer B.Cu) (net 8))
 (segment (start 204.520799 103.631999) (end 207.645001 106.756201) (width 0.3048) (layer B.Cu) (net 8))
 (segment (start 133.35 100.33) (end 141.6812 108.6612) (width 0.3048) (layer B.Cu) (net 10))
 (segment (start 141.6812 108.6612) (end 158.75 108.6612) (width 0.3048) (layer B.Cu) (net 10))
 (segment (start 163.656262 99.695) (end 218.7702 99.695) (width 1.27) (layer F.Cu) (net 13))
 (segment (start 218.7702 99.695) (end 221.9452 96.52) (width 1.27) (layer F.Cu) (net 13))
 (segment (start 123.19 110.49) (end 123.19 111.603551) (width 1.27) (layer F.Cu) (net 13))
 (segment (start 123.19 111.603551) (end 124.010912 112.424463) (width 1.27) (layer F.Cu) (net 13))
 (segment (start 124.010912 112.424463) (end 150.926799 112.424463) (width 1.27) (layer F.Cu) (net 13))
 (segment (start 150.926799 112.424463) (end 163.656262 99.695) (width 1.27) (layer F.Cu) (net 13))
 (segment (start 221.9452 96.52) (end 144.78 96.52) (width 1.27) (layer B.Cu) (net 13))
 (segment (start 144.78 96.52) (end 142.24 93.98) (width 1.27) (layer B.Cu) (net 13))
 (segment (start 118.11 110.49) (end 118.11 111.603551) (width 1.27) (layer F.Cu) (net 13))
 (segment (start 118.11 111.603551) (end 118.62205 112.115601) (width 1.27) (layer F.Cu) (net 13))
 (segment (start 118.62205 112.115601) (end 121.564399 112.115601) (width 1.27) (layer F.Cu) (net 13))
 (segment (start 121.564399 112.115601) (end 122.402601 111.277399) (width 1.27) (layer F.Cu) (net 13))
 (segment (start 122.402601 111.277399) (end 123.19 110.49) (width 1.27) (layer F.Cu) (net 13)))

